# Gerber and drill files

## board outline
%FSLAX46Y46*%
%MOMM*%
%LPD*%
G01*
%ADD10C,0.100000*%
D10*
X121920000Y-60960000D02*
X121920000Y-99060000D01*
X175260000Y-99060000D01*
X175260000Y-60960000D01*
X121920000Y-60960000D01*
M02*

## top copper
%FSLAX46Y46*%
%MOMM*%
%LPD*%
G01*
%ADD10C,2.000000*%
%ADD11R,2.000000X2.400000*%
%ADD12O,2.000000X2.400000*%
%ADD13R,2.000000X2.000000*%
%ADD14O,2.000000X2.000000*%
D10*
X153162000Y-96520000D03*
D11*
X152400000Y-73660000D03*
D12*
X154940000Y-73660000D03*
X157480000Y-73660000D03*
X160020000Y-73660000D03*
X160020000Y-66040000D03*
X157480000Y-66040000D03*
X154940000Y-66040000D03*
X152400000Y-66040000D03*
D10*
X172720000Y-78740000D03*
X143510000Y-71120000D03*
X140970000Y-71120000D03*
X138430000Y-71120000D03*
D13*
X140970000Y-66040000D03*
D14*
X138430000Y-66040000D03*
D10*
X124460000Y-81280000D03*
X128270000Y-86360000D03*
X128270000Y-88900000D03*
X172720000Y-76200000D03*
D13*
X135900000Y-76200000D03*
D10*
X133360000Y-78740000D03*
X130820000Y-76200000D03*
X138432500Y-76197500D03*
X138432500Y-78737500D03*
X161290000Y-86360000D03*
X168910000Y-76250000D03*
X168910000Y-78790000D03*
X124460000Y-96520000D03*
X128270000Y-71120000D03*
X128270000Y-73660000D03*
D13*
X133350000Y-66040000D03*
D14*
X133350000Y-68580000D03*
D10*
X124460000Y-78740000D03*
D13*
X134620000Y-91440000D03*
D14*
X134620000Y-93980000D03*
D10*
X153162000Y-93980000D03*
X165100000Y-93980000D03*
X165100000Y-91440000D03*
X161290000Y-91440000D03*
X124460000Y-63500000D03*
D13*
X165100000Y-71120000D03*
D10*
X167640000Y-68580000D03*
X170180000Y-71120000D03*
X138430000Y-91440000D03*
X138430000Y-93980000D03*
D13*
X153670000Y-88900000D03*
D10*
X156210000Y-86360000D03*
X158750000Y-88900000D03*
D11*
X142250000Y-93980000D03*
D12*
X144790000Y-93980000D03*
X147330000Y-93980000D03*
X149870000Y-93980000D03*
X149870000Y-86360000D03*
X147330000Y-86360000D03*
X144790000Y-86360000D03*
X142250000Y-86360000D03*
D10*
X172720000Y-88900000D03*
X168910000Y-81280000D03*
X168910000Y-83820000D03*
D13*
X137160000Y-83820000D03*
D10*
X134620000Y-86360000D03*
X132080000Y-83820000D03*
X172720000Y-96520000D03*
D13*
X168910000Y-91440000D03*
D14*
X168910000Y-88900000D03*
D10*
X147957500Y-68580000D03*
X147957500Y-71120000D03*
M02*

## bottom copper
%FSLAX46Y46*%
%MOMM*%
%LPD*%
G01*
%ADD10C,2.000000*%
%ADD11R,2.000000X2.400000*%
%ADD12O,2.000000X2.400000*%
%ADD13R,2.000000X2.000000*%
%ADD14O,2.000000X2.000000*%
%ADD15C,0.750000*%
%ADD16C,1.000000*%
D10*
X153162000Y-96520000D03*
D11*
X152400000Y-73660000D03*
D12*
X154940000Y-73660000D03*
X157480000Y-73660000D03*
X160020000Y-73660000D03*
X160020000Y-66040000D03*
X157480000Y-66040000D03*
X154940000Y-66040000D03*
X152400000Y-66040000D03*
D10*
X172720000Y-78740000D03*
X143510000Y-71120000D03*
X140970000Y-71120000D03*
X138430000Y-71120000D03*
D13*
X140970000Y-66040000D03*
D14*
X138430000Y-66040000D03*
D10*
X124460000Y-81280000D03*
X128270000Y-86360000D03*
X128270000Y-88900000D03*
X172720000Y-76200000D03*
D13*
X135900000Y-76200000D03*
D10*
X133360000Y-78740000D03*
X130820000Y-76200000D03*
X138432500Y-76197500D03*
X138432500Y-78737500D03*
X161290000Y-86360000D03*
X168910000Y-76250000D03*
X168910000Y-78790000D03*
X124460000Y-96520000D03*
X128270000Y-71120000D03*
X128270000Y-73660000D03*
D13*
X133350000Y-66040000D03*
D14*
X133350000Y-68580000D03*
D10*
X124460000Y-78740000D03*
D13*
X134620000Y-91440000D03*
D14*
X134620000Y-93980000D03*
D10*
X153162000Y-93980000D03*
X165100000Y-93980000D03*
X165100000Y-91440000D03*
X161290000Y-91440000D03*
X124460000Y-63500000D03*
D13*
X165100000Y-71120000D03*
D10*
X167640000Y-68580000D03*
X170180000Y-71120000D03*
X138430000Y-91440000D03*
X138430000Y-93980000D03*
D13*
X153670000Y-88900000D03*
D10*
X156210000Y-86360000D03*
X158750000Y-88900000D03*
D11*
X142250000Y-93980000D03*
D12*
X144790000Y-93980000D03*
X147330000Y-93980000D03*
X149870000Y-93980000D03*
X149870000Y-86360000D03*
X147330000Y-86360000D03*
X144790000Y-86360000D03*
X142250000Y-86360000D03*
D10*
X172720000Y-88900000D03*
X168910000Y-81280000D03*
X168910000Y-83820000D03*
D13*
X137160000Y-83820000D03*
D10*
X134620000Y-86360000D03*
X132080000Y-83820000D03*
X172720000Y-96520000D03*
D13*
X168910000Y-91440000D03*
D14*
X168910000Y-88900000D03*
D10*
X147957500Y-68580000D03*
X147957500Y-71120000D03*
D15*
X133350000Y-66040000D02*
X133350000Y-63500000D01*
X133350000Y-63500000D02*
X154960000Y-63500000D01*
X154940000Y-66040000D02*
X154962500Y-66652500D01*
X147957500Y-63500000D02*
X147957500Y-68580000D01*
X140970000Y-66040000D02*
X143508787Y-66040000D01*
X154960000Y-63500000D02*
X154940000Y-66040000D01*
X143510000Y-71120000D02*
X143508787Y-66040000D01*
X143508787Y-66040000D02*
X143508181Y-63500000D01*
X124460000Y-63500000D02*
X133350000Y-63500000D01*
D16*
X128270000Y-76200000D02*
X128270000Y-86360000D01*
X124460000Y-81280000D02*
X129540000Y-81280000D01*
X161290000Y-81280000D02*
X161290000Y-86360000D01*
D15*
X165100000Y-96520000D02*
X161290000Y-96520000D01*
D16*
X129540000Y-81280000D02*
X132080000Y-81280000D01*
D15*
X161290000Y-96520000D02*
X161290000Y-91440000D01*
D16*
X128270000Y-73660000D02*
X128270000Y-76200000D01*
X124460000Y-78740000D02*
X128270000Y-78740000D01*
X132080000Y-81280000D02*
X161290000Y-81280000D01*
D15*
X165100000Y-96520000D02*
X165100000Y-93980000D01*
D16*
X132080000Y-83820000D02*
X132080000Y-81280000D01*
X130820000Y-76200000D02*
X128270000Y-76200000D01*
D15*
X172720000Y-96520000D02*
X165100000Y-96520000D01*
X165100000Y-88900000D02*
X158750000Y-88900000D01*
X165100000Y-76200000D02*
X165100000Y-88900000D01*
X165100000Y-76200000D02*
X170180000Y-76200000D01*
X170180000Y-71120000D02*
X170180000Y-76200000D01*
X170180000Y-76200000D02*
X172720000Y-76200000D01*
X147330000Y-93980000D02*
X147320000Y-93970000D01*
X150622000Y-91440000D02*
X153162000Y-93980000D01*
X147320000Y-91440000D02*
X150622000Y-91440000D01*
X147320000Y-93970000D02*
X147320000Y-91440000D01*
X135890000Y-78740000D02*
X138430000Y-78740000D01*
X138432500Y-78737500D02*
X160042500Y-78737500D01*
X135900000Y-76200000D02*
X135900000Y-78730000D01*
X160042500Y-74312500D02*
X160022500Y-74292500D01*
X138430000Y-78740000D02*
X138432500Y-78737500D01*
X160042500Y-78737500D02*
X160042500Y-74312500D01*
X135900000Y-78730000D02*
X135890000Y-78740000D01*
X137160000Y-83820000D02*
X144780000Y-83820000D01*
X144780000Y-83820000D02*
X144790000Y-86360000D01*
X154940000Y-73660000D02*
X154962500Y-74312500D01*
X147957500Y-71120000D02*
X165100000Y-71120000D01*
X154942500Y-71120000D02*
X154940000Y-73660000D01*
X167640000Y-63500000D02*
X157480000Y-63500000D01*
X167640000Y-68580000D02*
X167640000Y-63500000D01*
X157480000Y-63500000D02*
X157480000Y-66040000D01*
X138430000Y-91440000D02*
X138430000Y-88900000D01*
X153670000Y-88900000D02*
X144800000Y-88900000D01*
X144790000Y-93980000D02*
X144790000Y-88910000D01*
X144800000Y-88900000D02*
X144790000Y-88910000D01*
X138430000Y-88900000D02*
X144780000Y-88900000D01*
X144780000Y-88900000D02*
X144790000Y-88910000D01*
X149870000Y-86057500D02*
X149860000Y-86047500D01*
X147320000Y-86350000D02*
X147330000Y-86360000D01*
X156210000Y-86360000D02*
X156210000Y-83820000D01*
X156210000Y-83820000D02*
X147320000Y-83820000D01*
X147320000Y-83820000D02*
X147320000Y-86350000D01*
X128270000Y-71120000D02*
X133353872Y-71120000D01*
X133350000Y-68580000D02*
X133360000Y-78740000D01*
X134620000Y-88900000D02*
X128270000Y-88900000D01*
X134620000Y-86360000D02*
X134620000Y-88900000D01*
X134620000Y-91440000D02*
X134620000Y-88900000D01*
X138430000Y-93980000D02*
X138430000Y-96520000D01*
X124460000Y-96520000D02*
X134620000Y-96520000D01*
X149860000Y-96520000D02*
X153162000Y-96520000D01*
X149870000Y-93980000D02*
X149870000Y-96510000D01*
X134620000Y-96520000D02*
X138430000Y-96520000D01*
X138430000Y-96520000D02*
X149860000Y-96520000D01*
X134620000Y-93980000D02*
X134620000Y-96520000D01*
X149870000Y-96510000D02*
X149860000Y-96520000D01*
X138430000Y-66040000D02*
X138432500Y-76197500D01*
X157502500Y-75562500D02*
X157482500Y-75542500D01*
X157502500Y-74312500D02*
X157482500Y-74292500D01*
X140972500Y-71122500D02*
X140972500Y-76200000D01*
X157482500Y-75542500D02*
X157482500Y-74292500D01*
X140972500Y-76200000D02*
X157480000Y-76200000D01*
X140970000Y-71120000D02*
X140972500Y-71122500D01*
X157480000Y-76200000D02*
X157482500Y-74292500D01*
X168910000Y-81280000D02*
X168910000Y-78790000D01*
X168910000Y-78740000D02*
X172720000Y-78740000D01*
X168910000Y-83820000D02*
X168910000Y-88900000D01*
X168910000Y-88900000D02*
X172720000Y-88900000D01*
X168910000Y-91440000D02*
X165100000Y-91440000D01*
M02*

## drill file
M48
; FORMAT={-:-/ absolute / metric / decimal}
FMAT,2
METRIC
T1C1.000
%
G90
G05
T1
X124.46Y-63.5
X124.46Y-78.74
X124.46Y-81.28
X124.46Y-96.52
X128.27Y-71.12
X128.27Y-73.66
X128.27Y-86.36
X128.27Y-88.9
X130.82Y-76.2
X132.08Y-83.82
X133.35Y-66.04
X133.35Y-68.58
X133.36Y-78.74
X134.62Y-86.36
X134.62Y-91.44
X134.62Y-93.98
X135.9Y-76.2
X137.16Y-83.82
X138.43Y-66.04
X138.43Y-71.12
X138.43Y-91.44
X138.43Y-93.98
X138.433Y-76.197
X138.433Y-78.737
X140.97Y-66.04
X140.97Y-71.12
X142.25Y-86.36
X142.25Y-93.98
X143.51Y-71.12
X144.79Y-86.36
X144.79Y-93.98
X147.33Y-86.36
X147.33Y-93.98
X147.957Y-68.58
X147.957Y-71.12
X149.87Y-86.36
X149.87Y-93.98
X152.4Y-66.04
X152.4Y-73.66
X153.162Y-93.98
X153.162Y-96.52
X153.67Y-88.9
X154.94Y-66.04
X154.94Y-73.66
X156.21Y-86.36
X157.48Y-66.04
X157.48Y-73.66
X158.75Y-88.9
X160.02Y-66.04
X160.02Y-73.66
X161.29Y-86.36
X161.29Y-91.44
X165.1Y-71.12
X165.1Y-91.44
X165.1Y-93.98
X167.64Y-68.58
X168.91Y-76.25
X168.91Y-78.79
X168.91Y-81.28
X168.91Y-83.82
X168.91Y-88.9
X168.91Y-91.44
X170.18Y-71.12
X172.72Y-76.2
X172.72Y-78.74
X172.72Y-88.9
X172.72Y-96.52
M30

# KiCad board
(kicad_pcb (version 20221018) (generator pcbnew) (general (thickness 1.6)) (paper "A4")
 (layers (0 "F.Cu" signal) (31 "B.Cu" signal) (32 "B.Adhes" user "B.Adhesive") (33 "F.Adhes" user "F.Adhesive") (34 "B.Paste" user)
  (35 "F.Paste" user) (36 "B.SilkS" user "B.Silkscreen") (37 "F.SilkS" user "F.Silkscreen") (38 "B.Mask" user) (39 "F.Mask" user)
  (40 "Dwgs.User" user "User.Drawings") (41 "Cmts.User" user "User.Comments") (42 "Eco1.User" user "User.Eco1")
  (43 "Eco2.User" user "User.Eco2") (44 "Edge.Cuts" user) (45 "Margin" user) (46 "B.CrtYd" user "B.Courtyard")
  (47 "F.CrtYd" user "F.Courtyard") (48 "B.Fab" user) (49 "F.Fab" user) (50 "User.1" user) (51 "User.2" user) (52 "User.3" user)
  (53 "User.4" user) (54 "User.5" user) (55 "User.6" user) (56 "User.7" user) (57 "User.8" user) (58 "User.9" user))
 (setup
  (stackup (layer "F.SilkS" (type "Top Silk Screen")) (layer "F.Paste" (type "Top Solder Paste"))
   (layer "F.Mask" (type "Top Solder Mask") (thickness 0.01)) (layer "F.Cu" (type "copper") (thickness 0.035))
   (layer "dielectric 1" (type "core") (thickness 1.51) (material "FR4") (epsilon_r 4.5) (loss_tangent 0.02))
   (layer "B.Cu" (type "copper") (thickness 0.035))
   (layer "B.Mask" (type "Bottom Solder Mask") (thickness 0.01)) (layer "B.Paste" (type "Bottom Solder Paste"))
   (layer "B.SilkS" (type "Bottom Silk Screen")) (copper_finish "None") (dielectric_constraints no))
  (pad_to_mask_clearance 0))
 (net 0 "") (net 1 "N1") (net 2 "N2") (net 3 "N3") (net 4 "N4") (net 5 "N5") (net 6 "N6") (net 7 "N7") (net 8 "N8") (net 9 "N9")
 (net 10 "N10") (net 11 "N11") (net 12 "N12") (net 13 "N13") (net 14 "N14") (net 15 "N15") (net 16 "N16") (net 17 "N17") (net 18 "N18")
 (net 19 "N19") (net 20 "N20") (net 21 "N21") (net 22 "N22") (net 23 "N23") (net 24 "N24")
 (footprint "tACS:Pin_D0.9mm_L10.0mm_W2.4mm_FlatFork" (layer "F.Cu") (at 153.162 96.52)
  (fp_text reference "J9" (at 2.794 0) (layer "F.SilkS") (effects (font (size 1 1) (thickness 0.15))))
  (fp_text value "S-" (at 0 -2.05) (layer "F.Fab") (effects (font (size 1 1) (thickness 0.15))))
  (pad "1" thru_hole circle (at 0 0) (size 2 2) (drill 1) (layers "*.Cu" "*.Mask") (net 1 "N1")))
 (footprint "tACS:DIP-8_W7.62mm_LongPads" (layer "F.Cu") (at 152.4 73.66 90)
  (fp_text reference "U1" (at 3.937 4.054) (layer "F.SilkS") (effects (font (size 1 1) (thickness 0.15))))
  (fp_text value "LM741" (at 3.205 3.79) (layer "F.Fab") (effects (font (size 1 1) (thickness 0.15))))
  (pad "1" thru_hole rect (at 0 0 90) (size 2.4 2) (drill 1) (layers "*.Cu" "*.Mask") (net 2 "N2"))
  (pad "2" thru_hole oval (at 0 2.54 90) (size 2.4 2) (drill 1) (layers "*.Cu" "*.Mask") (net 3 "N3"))
  (pad "3" thru_hole oval (at 0 5.08 90) (size 2.4 2) (drill 1) (layers "*.Cu" "*.Mask") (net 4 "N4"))
  (pad "4" thru_hole oval (at 0 7.62 90) (size 2.4 2) (drill 1) (layers "*.Cu" "*.Mask") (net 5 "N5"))
  (pad "5" thru_hole oval (at 7.62 7.62 90) (size 2.4 2) (drill 1) (layers "*.Cu" "*.Mask") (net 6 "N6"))
  (pad "6" thru_hole oval (at 7.62 5.08 90) (size 2.4 2) (drill 1) (layers "*.Cu" "*.Mask") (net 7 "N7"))
  (pad "7" thru_hole oval (at 7.62 2.54 90) (size 2.4 2) (drill 1) (layers "*.Cu" "*.Mask") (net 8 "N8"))
  (pad "8" thru_hole oval (at 7.62 0 90) (size 2.4 2) (drill 1) (layers "*.Cu" "*.Mask") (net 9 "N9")))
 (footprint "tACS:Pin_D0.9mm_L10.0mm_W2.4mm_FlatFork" (layer "F.Cu") (at 172.72 78.74)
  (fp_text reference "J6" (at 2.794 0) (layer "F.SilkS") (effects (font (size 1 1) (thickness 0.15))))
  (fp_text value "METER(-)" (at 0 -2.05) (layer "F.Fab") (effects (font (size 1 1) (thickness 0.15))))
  (pad "1" thru_hole circle (at 0 0) (size 2 2) (drill 1) (layers "*.Cu" "*.Mask") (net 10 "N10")))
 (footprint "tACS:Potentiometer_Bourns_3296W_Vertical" (layer "F.Cu") (at 143.51 71.12)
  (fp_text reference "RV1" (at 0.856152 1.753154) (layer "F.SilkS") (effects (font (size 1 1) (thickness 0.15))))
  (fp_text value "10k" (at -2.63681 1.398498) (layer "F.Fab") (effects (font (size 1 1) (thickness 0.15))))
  (pad "1" thru_hole circle (at 0 0) (size 2 2) (drill 1) (layers "*.Cu" "*.Mask") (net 8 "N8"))
  (pad "2" thru_hole circle (at -2.54 0) (size 2 2) (drill 1) (layers "*.Cu" "*.Mask") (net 4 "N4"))
  (pad "3" thru_hole circle (at -5.08 0) (size 2 2) (drill 1) (layers "*.Cu" "*.Mask") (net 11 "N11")))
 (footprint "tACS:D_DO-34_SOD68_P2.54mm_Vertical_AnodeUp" (layer "F.Cu") (at 140.97 66.04 180)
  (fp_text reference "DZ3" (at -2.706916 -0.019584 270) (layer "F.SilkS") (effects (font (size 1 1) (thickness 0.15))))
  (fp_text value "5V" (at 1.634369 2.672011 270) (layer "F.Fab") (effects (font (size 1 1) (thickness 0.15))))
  (pad "1" thru_hole rect (at 0 0 180) (size 2 2) (drill 1) (layers "*.Cu" "*.Mask") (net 8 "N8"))
  (pad "2" thru_hole oval (at 2.54 0 180) (size 2 2) (drill 1) (layers "*.Cu" "*.Mask") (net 11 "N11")))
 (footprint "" (layer "F.Cu") (at 124.46 81.28)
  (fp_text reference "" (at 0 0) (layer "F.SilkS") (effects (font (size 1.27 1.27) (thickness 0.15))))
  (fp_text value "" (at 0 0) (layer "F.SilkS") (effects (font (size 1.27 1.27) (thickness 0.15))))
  (pad "1" thru_hole circle (at 0 0) (size 2 2) (drill 1) (layers "*.Cu" "*.Mask") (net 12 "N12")))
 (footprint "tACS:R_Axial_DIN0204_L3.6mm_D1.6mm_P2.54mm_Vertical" (layer "F.Cu") (at 128.27 86.36 -90)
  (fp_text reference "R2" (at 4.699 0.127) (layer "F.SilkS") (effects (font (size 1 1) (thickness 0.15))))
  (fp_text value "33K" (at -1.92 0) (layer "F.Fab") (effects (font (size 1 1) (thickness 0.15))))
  (pad "1" thru_hole circle (at 0 0 270) (size 2 2) (drill 1) (layers "*.Cu" "*.Mask") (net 12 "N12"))
  (pad "2" thru_hole circle (at 2.54 0 270) (size 2 2) (drill 1) (layers "*.Cu" "*.Mask") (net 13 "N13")))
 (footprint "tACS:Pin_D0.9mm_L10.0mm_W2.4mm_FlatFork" (layer "F.Cu") (at 172.72 76.2)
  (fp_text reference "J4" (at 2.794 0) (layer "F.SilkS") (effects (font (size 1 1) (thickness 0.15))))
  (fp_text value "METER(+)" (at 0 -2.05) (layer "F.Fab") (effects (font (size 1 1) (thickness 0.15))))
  (pad "1" thru_hole circle (at 0 0) (size 2 2) (drill 1) (layers "*.Cu" "*.Mask") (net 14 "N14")))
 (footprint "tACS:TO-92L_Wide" (layer "F.Cu") (at 135.9 76.2 180)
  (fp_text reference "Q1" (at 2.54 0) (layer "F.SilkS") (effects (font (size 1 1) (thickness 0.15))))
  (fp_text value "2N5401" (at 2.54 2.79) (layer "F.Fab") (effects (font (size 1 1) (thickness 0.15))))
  (pad "1" thru_hole rect (at 0 0 180) (size 2 2) (drill 1) (layers "*.Cu" "*.Mask") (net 5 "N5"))
  (pad "2" thru_hole circle (at 2.54 -2.54 180) (size 2 2) (drill 1) (layers "*.Cu" "*.Mask") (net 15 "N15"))
  (pad "3" thru_hole circle (at 5.08 0 180) (size 2 2) (drill 1) (layers "*.Cu" "*.Mask") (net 12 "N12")))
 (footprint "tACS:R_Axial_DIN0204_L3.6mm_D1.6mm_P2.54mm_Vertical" (layer "F.Cu") (at 138.4325 76.1975 -90)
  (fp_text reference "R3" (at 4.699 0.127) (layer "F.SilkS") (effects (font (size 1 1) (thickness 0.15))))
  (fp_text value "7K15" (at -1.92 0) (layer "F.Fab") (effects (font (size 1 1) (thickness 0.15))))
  (pad "1" thru_hole circle (at 0 0 270) (size 2 2) (drill 1) (layers "*.Cu" "*.Mask") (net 11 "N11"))
  (pad "2" thru_hole circle (at 2.54 0 270) (size 2 2) (drill 1) (layers "*.Cu" "*.Mask") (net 5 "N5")))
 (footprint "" (layer "F.Cu") (at 161.29 86.36)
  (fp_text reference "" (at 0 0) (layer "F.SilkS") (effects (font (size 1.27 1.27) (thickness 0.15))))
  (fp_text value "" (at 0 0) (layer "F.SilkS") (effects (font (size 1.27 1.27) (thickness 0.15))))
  (pad "1" thru_hole circle (at 0 0) (size 2 2) (drill 1) (layers "*.Cu" "*.Mask") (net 12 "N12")))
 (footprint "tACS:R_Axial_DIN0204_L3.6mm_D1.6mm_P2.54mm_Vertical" (layer "F.Cu") (at 168.91 76.25 -90)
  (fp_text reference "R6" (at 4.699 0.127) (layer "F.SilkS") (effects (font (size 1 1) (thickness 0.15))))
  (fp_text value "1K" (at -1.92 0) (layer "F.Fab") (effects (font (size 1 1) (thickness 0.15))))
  (pad "1" thru_hole circle (at 0 0 270) (size 2 2) (drill 1) (layers "*.Cu" "*.Mask") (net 14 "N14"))
  (pad "2" thru_hole circle (at 2.54 0 270) (size 2 2) (drill 1) (layers "*.Cu" "*.Mask") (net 10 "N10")))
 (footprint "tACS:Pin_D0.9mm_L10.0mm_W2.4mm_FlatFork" (layer "F.Cu") (at 124.46 96.52)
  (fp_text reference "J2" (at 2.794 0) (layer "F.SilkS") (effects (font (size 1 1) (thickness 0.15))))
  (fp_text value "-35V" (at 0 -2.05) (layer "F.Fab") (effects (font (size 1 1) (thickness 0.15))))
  (pad "1" thru_hole circle (at 0 0) (size 2 2) (drill 1) (layers "*.Cu" "*.Mask") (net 1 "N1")))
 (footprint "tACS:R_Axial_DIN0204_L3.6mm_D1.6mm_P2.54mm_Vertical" (layer "F.Cu") (at 128.27 71.12 -90)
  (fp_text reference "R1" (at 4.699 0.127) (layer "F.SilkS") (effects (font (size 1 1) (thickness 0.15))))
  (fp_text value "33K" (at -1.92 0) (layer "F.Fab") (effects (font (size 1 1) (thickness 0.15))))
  (pad "1" thru_hole circle (at 0 0 270) (size 2 2) (drill 1) (layers "*.Cu" "*.Mask") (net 15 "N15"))
  (pad "2" thru_hole circle (at 2.54 0 270) (size 2 2) (drill 1) (layers "*.Cu" "*.Mask") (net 12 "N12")))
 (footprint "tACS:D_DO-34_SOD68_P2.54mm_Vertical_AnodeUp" (layer "F.Cu") (at 133.35 66.04 -90)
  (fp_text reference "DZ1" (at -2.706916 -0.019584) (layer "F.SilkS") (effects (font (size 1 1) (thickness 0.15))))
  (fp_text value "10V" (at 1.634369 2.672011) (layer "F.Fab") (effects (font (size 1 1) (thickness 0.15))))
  (pad "1" thru_hole rect (at 0 0 270) (size 2 2) (drill 1) (layers "*.Cu" "*.Mask") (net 8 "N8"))
  (pad "2" thru_hole oval (at 2.54 0 270) (size 2 2) (drill 1) (layers "*.Cu" "*.Mask") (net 15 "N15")))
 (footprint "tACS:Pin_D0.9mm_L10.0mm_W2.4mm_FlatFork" (layer "F.Cu") (at 124.46 78.74)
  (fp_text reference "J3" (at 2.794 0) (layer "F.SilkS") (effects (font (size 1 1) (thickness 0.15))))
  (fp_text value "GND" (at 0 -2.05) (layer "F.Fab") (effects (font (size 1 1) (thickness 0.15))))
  (pad "1" thru_hole circle (at 0 0) (size 2 2) (drill 1) (layers "*.Cu" "*.Mask") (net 12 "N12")))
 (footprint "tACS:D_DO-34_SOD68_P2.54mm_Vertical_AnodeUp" (layer "F.Cu") (at 134.62 91.44 -90)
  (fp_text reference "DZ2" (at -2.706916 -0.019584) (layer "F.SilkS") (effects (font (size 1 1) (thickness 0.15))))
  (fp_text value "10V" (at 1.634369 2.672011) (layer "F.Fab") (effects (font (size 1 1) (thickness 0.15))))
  (pad "1" thru_hole rect (at 0 0 270) (size 2 2) (drill 1) (layers "*.Cu" "*.Mask") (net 13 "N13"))
  (pad "2" thru_hole oval (at 2.54 0 270) (size 2 2) (drill 1) (layers "*.Cu" "*.Mask") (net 1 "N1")))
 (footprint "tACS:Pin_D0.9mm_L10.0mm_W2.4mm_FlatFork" (layer "F.Cu") (at 153.162 93.98)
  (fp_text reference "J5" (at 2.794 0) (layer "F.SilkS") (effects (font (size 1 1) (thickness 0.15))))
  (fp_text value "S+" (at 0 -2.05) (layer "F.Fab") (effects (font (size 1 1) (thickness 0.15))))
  (pad "1" thru_hole circle (at 0 0) (size 2 2) (drill 1) (layers "*.Cu" "*.Mask") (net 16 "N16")))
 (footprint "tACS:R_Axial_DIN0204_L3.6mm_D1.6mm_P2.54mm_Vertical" (layer "F.Cu") (at 165.1 93.98 90)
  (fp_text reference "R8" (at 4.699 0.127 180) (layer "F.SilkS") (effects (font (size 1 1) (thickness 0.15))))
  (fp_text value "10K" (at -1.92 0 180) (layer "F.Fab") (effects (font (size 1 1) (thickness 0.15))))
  (pad "1" thru_hole circle (at 0 0 90) (size 2 2) (drill 1) (layers "*.Cu" "*.Mask") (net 12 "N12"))
  (pad "2" thru_hole circle (at 2.54 0 90) (size 2 2) (drill 1) (layers "*.Cu" "*.Mask") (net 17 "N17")))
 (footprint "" (layer "F.Cu") (at 161.29 91.44)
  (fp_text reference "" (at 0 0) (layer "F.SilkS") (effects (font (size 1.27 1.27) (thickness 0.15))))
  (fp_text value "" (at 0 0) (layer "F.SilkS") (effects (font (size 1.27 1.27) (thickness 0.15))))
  (pad "1" thru_hole circle (at 0 0) (size 2 2) (drill 1) (layers "*.Cu" "*.Mask") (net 12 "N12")))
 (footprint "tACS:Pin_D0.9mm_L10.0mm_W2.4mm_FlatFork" (layer "F.Cu") (at 124.46 63.5)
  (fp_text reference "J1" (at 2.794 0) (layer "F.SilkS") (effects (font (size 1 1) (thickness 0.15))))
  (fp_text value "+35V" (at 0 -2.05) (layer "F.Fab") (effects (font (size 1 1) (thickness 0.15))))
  (pad "1" thru_hole circle (at 0 0) (size 2 2) (drill 1) (layers "*.Cu" "*.Mask") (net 8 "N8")))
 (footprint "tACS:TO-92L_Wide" (layer "F.Cu") (at 165.1 71.12)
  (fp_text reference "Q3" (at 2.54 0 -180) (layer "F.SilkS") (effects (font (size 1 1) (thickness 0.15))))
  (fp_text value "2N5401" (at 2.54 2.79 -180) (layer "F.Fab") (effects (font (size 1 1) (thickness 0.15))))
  (pad "1" thru_hole rect (at 0 0) (size 2 2) (drill 1) (layers "*.Cu" "*.Mask") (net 3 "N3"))
  (pad "2" thru_hole circle (at 2.54 -2.54) (size 2 2) (drill 1) (layers "*.Cu" "*.Mask") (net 7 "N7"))
  (pad "3" thru_hole circle (at 5.08 0) (size 2 2) (drill 1) (layers "*.Cu" "*.Mask") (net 14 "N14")))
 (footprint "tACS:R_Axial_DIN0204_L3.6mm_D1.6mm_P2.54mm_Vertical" (layer "F.Cu") (at 138.43 91.44 -90)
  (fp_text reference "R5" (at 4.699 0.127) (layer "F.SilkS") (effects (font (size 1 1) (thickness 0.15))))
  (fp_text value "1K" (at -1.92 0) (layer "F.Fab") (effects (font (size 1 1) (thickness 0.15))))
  (pad "1" thru_hole circle (at 0 0 270) (size 2 2) (drill 1) (layers "*.Cu" "*.Mask") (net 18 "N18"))
  (pad "2" thru_hole circle (at 2.54 0 270) (size 2 2) (drill 1) (layers "*.Cu" "*.Mask") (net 1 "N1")))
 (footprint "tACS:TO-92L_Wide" (layer "F.Cu") (at 153.67 88.9)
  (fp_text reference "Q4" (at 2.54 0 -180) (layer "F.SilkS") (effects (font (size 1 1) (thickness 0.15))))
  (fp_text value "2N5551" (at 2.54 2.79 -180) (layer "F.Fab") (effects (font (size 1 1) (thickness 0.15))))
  (pad "1" thru_hole rect (at 0 0) (size 2 2) (drill 1) (layers "*.Cu" "*.Mask") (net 18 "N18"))
  (pad "2" thru_hole circle (at 2.54 -2.54) (size 2 2) (drill 1) (layers "*.Cu" "*.Mask") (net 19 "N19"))
  (pad "3" thru_hole circle (at 5.08 0) (size 2 2) (drill 1) (layers "*.Cu" "*.Mask") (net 14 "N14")))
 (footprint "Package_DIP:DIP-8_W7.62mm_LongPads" (layer "F.Cu") (at 142.25 93.98 90)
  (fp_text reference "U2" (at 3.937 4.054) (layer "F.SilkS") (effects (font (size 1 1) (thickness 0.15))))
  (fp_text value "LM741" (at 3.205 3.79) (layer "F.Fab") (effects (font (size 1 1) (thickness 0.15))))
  (pad "1" thru_hole rect (at 0 0 90) (size 2.4 2) (drill 1) (layers "*.Cu" "*.Mask") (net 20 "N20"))
  (pad "2" thru_hole oval (at 0 2.54 90) (size 2.4 2) (drill 1) (layers "*.Cu" "*.Mask") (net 18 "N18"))
  (pad "3" thru_hole oval (at 0 5.08 90) (size 2.4 2) (drill 1) (layers "*.Cu" "*.Mask") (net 16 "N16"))
  (pad "4" thru_hole oval (at 0 7.62 90) (size 2.4 2) (drill 1) (layers "*.Cu" "*.Mask") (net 1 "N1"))
  (pad "5" thru_hole oval (at 7.62 7.62 90) (size 2.4 2) (drill 1) (layers "*.Cu" "*.Mask") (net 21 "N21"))
  (pad "6" thru_hole oval (at 7.62 5.08 90) (size 2.4 2) (drill 1) (layers "*.Cu" "*.Mask") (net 19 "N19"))
  (pad "7" thru_hole oval (at 7.62 2.54 90) (size 2.4 2) (drill 1) (layers "*.Cu" "*.Mask") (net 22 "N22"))
  (pad "8" thru_hole oval (at 7.62 0 90) (size 2.4 2) (drill 1) (layers "*.Cu" "*.Mask") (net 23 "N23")))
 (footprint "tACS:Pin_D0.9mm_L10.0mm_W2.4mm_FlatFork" (layer "F.Cu") (at 172.72 88.9)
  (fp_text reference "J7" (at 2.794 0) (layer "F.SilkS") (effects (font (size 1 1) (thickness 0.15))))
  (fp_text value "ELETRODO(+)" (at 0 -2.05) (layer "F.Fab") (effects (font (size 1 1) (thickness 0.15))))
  (pad "1" thru_hole circle (at 0 0) (size 2 2) (drill 1) (layers "*.Cu" "*.Mask") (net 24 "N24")))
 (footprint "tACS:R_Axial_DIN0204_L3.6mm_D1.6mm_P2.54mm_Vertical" (layer "F.Cu") (at 168.91 81.28 -90)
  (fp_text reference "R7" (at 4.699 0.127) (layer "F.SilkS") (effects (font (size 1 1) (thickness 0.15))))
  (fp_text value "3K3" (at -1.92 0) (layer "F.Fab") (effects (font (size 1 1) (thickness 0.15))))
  (pad "1" thru_hole circle (at 0 0 270) (size 2 2) (drill 1) (layers "*.Cu" "*.Mask") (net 10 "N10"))
  (pad "2" thru_hole circle (at 2.54 0 270) (size 2 2) (drill 1) (layers "*.Cu" "*.Mask") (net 24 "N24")))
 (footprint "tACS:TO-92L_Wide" (layer "F.Cu") (at 137.16 83.82 180)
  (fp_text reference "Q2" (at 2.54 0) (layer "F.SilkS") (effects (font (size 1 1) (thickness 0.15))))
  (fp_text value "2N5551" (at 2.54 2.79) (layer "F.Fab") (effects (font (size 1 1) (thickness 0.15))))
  (pad "1" thru_hole rect (at 0 0 180) (size 2 2) (drill 1) (layers "*.Cu" "*.Mask") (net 22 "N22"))
  (pad "2" thru_hole circle (at 2.54 -2.54 180) (size 2 2) (drill 1) (layers "*.Cu" "*.Mask") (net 13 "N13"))
  (pad "3" thru_hole circle (at 5.08 0 180) (size 2 2) (drill 1) (layers "*.Cu" "*.Mask") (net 12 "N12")))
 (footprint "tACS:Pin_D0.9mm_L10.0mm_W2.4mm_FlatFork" (layer "F.Cu") (at 172.72 96.52)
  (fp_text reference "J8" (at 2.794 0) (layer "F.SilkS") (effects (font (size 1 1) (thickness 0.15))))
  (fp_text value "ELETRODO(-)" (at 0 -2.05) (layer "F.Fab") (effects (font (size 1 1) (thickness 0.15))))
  (pad "1" thru_hole circle (at 0 0) (size 2 2) (drill 1) (layers "*.Cu" "*.Mask") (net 12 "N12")))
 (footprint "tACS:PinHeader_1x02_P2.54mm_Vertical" (layer "F.Cu") (at 168.91 91.44 180)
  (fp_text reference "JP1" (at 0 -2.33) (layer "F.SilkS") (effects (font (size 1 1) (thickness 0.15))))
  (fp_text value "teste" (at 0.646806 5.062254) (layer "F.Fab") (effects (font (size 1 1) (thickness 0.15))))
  (pad "1" thru_hole rect (at 0 0 180) (size 2 2) (drill 1) (layers "*.Cu" "*.Mask") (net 17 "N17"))
  (pad "2" thru_hole oval (at 0 2.54 180) (size 2 2) (drill 1) (layers "*.Cu" "*.Mask") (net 24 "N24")))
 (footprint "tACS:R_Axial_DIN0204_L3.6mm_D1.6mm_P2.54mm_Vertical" (layer "F.Cu") (at 147.9575 68.58 -90)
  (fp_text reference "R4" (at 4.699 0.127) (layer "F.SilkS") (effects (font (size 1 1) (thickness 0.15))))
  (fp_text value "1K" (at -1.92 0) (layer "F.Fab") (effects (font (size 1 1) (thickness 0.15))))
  (pad "1" thru_hole circle (at 0 0 270) (size 2 2) (drill 1) (layers "*.Cu" "*.Mask") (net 8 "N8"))
  (pad "2" thru_hole circle (at 2.54 0 270) (size 2 2) (drill 1) (layers "*.Cu" "*.Mask") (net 3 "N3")))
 (gr_poly
  (pts (xy 121.92 60.96) (xy 121.92 99.06) (xy 175.26 99.06) (xy 175.26 60.96)) (stroke (width 0.1) (type solid)) (fill none)
  (layer "Edge.Cuts"))
 (segment (start 133.35 66.04) (end 133.35 63.5) (width 0.75) (layer "B.Cu") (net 8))
 (segment (start 133.35 63.5) (end 154.96 63.5) (width 0.75) (layer "B.Cu") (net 8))
 (segment (start 154.94 66.04) (end 154.9625 66.6525) (width 0.75) (layer "B.Cu") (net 8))
 (segment (start 147.9575 63.5) (end 147.9575 68.58) (width 0.75) (layer "B.Cu") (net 8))
 (segment (start 140.97 66.04) (end 143.508787 66.04) (width 0.75) (layer "B.Cu") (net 8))
 (segment (start 154.96 63.5) (end 154.94 66.04) (width 0.75) (layer "B.Cu") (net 8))
 (segment (start 143.51 71.12) (end 143.508787 66.04) (width 0.75) (layer "B.Cu") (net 8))
 (segment (start 143.508787 66.04) (end 143.508181 63.5) (width 0.75) (layer "B.Cu") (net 8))
 (segment (start 124.46 63.5) (end 133.35 63.5) (width 0.75) (layer "B.Cu") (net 8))
 (segment (start 128.27 76.2) (end 128.27 86.36) (width 1) (layer "B.Cu") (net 12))
 (segment (start 124.46 81.28) (end 129.54 81.28) (width 1) (layer "B.Cu") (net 12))
 (segment (start 161.29 81.28) (end 161.29 86.36) (width 1) (layer "B.Cu") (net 12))
 (segment (start 165.1 96.52) (end 161.29 96.52) (width 0.75) (layer "B.Cu") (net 12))
 (segment (start 129.54 81.28) (end 132.08 81.28) (width 1) (layer "B.Cu") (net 12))
 (segment (start 161.29 96.52) (end 161.29 91.44) (width 0.75) (layer "B.Cu") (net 12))
 (segment (start 128.27 73.66) (end 128.27 76.2) (width 1) (layer "B.Cu") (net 12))
 (segment (start 124.46 78.74) (end 128.27 78.74) (width 1) (layer "B.Cu") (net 12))
 (segment (start 132.08 81.28) (end 161.29 81.28) (width 1) (layer "B.Cu") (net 12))
 (segment (start 165.1 96.52) (end 165.1 93.98) (width 0.75) (layer "B.Cu") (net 12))
 (segment (start 132.08 83.82) (end 132.08 81.28) (width 1) (layer "B.Cu") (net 12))
 (segment (start 130.82 76.2) (end 128.27 76.2) (width 1) (layer "B.Cu") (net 12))
 (segment (start 172.72 96.52) (end 165.1 96.52) (width 0.75) (layer "B.Cu") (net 12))
 (segment (start 165.1 88.9) (end 158.75 88.9) (width 0.75) (layer "B.Cu") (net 14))
 (segment (start 165.1 76.2) (end 165.1 88.9) (width 0.75) (layer "B.Cu") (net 14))
 (segment (start 165.1 76.2) (end 170.18 76.2) (width 0.75) (layer "B.Cu") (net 14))
 (segment (start 170.18 71.12) (end 170.18 76.2) (width 0.75) (layer "B.Cu") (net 14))
 (segment (start 170.18 76.2) (end 172.72 76.2) (width 0.75) (layer "B.Cu") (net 14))
 (segment (start 147.33 93.98) (end 147.32 93.97) (width 0.75) (layer "B.Cu") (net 16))
 (segment (start 150.622 91.44) (end 153.162 93.98) (width 0.75) (layer "B.Cu") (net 16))
 (segment (start 147.32 91.44) (end 150.622 91.44) (width 0.75) (layer "B.Cu") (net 16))
 (segment (start 147.32 93.97) (end 147.32 91.44) (width 0.75) (layer "B.Cu") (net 16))
 (segment (start 135.89 78.74) (end 138.43 78.74) (width 0.75) (layer "B.Cu") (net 5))
 (segment (start 138.4325 78.7375) (end 160.0425 78.7375) (width 0.75) (layer "B.Cu") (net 5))
 (segment (start 135.9 76.2) (end 135.9 78.73) (width 0.75) (layer "B.Cu") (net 5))
 (segment (start 160.0425 74.3125) (end 160.0225 74.2925) (width 0.75) (layer "B.Cu") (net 5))
 (segment (start 138.43 78.74) (end 138.4325 78.7375) (width 0.75) (layer "B.Cu") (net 5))
 (segment (start 160.0425 78.7375) (end 160.0425 74.3125) (width 0.75) (layer "B.Cu") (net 5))
 (segment (start 135.9 78.73) (end 135.89 78.74) (width 0.75) (layer "B.Cu") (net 5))
 (segment (start 137.16 83.82) (end 144.78 83.82) (width 0.75) (layer "B.Cu") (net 22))
 (segment (start 144.78 83.82) (end 144.79 86.36) (width 0.75) (layer "B.Cu") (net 22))
 (segment (start 154.94 73.66) (end 154.9625 74.3125) (width 0.75) (layer "B.Cu") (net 3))
 (segment (start 147.9575 71.12) (end 165.1 71.12) (width 0.75) (layer "B.Cu") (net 3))
 (segment (start 154.9425 71.12) (end 154.94 73.66) (width 0.75) (layer "B.Cu") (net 3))
 (segment (start 167.64 63.5) (end 157.48 63.5) (width 0.75) (layer "B.Cu") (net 7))
 (segment (start 167.64 68.58) (end 167.64 63.5) (width 0.75) (layer "B.Cu") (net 7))
 (segment (start 157.48 63.5) (end 157.48 66.04) (width 0.75) (layer "B.Cu") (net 7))
 (segment (start 138.43 91.44) (end 138.43 88.9) (width 0.75) (layer "B.Cu") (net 18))
 (segment (start 153.67 88.9) (end 144.8 88.9) (width 0.75) (layer "B.Cu") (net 18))
 (segment (start 144.79 93.98) (end 144.79 88.91) (width 0.75) (layer "B.Cu") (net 18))
 (segment (start 144.8 88.9) (end 144.79 88.91) (width 0.75) (layer "B.Cu") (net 18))
 (segment (start 138.43 88.9) (end 144.78 88.9) (width 0.75) (layer "B.Cu") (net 18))
 (segment (start 144.78 88.9) (end 144.79 88.91) (width 0.75) (layer "B.Cu") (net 18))
 (segment (start 149.87 86.0575) (end 149.86 86.0475) (width 0.75) (layer "B.Cu") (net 21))
 (segment (start 147.32 86.35) (end 147.33 86.36) (width 0.75) (layer "B.Cu") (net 19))
 (segment (start 156.21 86.36) (end 156.21 83.82) (width 0.75) (layer "B.Cu") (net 19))
 (segment (start 156.21 83.82) (end 147.32 83.82) (width 0.75) (layer "B.Cu") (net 19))
 (segment (start 147.32 83.82) (end 147.32 86.35) (width 0.75) (layer "B.Cu") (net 19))
 (segment (start 128.27 71.12) (end 133.353872 71.12) (width 0.75) (layer "B.Cu") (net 15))
 (segment (start 133.35 68.58) (end 133.36 78.74) (width 0.75) (layer "B.Cu") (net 15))
 (segment (start 134.62 88.9) (end 128.27 88.9) (width 0.75) (layer "B.Cu") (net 13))
 (segment (start 134.62 86.36) (end 134.62 88.9) (width 0.75) (layer "B.Cu") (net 13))
 (segment (start 134.62 91.44) (end 134.62 88.9) (width 0.75) (layer "B.Cu") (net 13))
 (segment (start 138.43 93.98) (end 138.43 96.52) (width 0.75) (layer "B.Cu") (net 1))
 (segment (start 124.46 96.52) (end 134.62 96.52) (width 0.75) (layer "B.Cu") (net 1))
 (segment (start 149.86 96.52) (end 153.162 96.52) (width 0.75) (layer "B.Cu") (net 1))
 (segment (start 149.87 93.98) (end 149.87 96.51) (width 0.75) (layer "B.Cu") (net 1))
 (segment (start 134.62 96.52) (end 138.43 96.52) (width 0.75) (layer "B.Cu") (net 1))
 (segment (start 138.43 96.52) (end 149.86 96.52) (width 0.75) (layer "B.Cu") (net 1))
 (segment (start 134.62 93.98) (end 134.62 96.52) (width 0.75) (layer "B.Cu") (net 1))
 (segment (start 149.87 96.51) (end 149.86 96.52) (width 0.75) (layer "B.Cu") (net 1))
 (segment (start 138.43 66.04) (end 138.4325 76.1975) (width 0.75) (layer "B.Cu") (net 11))
 (segment (start 157.5025 75.5625) (end 157.4825 75.5425) (width 0.75) (layer "B.Cu") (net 4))
 (segment (start 157.5025 74.3125) (end 157.4825 74.2925) (width 0.75) (layer "B.Cu") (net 4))
 (segment (start 140.9725 71.1225) (end 140.9725 76.2) (width 0.75) (layer "B.Cu") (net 4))
 (segment (start 157.4825 75.5425) (end 157.4825 74.2925) (width 0.75) (layer "B.Cu") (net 4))
 (segment (start 140.9725 76.2) (end 157.48 76.2) (width 0.75) (layer "B.Cu") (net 4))
 (segment (start 140.97 71.12) (end 140.9725 71.1225) (width 0.75) (layer "B.Cu") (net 4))
 (segment (start 157.48 76.2) (end 157.4825 74.2925) (width 0.75) (layer "B.Cu") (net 4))
 (segment (start 168.91 81.28) (end 168.91 78.79) (width 0.75) (layer "B.Cu") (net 10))
 (segment (start 168.91 78.74) (end 172.72 78.74) (width 0.75) (layer "B.Cu") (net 10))
 (segment (start 168.91 83.82) (end 168.91 88.9) (width 0.75) (layer "B.Cu") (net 24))
 (segment (start 168.91 88.9) (end 172.72 88.9) (width 0.75) (layer "B.Cu") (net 24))
 (segment (start 168.91 91.44) (end 165.1 91.44) (width 0.75) (layer "B.Cu") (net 17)))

